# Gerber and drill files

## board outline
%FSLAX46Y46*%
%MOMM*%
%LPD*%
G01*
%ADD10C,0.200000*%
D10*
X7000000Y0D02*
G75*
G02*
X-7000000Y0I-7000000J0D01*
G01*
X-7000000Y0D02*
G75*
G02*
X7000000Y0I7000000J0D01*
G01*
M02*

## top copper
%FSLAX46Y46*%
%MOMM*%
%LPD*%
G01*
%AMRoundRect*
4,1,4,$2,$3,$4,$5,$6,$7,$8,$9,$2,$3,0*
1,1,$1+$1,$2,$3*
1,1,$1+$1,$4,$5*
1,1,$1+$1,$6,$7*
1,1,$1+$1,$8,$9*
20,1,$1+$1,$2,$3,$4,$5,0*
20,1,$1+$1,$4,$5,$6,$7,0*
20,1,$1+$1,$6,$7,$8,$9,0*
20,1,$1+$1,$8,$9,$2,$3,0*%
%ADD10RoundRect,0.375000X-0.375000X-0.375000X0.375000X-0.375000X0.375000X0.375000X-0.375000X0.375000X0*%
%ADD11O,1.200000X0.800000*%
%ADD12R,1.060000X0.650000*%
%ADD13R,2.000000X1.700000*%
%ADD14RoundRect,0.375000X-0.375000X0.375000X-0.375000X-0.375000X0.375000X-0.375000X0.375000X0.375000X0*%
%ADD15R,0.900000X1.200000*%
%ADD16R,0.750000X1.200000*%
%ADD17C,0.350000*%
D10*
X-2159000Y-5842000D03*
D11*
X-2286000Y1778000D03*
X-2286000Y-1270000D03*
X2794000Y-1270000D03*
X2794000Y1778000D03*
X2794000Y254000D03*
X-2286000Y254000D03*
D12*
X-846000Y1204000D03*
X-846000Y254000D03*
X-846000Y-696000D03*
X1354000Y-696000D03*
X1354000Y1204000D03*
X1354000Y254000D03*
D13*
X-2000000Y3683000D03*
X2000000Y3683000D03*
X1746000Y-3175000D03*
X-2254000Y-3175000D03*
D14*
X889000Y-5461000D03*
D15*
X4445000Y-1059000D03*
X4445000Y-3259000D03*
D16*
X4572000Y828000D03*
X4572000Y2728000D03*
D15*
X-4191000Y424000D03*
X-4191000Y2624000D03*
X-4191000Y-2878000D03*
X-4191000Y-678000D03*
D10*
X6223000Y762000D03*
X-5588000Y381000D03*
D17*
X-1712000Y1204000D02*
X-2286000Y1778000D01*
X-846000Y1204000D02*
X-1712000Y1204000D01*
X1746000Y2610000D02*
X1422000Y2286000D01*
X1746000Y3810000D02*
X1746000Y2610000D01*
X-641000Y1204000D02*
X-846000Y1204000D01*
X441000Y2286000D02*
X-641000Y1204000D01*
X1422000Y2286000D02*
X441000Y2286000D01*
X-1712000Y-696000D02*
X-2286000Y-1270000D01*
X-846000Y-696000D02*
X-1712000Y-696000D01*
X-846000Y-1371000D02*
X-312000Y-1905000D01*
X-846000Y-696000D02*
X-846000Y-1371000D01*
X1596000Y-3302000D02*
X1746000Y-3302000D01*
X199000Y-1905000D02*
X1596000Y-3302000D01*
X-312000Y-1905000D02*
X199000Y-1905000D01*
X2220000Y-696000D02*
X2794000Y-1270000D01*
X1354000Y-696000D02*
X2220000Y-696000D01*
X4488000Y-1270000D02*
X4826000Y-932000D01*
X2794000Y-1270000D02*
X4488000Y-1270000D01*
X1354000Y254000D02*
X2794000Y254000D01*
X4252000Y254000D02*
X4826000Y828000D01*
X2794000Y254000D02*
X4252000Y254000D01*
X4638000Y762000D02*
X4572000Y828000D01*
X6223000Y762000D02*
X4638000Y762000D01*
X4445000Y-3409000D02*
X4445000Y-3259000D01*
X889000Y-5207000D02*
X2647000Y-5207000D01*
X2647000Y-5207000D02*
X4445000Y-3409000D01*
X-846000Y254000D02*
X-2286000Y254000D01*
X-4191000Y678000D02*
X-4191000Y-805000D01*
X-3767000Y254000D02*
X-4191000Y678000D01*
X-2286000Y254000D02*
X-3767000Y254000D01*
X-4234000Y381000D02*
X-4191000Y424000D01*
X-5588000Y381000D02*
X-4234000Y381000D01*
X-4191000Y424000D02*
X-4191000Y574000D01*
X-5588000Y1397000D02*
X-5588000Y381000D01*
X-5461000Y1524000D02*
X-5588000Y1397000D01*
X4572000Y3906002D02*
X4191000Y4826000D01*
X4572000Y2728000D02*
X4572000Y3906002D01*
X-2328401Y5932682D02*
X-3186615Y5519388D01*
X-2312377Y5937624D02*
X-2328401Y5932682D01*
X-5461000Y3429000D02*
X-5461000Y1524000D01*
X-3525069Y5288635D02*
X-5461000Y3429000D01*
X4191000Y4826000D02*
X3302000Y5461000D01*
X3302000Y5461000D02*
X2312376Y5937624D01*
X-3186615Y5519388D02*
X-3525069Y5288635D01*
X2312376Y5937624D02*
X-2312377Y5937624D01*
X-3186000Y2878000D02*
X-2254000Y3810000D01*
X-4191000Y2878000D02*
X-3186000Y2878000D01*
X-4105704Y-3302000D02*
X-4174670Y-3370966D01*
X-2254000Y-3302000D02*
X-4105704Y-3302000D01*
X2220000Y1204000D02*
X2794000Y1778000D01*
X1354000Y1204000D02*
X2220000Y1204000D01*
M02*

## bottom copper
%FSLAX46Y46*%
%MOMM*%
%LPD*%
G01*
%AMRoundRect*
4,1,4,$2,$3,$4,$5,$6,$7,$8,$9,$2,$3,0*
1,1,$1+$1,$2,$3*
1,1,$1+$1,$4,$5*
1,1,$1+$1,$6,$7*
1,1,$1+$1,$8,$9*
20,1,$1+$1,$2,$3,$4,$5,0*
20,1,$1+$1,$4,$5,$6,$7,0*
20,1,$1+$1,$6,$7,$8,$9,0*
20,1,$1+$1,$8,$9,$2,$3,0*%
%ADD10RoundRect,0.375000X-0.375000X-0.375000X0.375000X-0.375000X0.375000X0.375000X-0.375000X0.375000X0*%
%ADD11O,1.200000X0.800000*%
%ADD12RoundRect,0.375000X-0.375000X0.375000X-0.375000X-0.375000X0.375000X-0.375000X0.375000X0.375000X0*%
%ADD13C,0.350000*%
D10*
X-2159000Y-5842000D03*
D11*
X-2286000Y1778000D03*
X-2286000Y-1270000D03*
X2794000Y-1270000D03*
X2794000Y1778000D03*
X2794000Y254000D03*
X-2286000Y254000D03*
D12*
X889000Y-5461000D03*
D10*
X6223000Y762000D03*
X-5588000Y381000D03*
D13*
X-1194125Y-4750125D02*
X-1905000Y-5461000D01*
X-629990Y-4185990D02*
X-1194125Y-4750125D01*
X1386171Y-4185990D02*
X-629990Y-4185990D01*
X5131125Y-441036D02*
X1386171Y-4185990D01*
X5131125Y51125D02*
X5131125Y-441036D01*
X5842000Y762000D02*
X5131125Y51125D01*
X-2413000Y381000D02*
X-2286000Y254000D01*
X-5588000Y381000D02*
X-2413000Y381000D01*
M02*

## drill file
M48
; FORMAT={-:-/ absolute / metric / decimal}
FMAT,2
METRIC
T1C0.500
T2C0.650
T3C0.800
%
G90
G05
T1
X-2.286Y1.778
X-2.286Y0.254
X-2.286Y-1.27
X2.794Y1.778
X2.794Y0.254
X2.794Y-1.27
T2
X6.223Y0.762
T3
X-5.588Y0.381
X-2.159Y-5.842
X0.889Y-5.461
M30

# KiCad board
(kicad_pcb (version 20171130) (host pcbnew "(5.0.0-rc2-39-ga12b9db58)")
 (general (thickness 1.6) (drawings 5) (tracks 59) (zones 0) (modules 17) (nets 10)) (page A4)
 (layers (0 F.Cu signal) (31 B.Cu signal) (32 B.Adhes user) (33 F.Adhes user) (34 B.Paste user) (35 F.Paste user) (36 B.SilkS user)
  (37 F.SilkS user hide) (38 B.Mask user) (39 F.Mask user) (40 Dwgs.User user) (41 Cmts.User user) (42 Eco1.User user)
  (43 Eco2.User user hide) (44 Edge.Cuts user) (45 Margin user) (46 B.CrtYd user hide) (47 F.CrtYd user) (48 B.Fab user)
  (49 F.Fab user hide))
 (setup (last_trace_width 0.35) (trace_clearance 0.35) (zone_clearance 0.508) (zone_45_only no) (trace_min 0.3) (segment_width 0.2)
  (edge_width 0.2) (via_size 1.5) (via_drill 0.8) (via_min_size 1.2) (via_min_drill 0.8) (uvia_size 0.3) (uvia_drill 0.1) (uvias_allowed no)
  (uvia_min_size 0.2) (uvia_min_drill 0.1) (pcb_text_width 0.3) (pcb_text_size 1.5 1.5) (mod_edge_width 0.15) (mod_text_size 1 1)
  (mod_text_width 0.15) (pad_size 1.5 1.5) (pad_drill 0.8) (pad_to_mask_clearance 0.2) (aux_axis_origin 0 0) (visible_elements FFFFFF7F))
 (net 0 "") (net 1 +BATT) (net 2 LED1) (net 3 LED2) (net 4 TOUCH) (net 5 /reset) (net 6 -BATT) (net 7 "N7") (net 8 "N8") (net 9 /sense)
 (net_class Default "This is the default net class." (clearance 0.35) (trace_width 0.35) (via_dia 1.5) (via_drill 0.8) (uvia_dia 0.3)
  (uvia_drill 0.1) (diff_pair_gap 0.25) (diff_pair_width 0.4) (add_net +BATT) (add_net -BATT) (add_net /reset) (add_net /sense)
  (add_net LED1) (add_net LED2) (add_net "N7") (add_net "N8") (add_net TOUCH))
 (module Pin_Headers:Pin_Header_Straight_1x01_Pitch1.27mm (layer F.Cu) (at -2.159 5.842)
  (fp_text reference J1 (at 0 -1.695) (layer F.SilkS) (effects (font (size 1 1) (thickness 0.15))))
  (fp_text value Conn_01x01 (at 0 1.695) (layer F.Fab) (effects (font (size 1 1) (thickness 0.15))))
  (pad 1 thru_hole roundrect (at 0 0) (size 1.5 1.5) (drill 0.8) (layers *.Cu *.Mask) (roundrect_rratio 0.25) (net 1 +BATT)))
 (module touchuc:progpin (layer F.Cu) (at -2.286 -1.778 90)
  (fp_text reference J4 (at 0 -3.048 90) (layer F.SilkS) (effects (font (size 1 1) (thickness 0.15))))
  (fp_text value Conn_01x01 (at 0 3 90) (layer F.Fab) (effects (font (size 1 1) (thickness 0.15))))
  (pad 1 thru_hole oval (at 0 0 90) (size 0.8 1.2) (drill 0.5) (layers *.Cu *.Mask) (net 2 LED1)))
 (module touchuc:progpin (layer F.Cu) (at -2.286 1.27 90)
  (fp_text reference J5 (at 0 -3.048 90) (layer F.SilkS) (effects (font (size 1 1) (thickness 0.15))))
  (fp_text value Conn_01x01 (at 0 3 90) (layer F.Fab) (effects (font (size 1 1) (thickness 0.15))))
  (pad 1 thru_hole oval (at 0 0 90) (size 0.8 1.2) (drill 0.5) (layers *.Cu *.Mask) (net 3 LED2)))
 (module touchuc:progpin (layer F.Cu) (at 2.794 1.27 90)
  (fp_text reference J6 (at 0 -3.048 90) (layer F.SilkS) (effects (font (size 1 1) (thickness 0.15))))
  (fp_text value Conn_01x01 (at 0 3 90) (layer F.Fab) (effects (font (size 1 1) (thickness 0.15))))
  (pad 1 thru_hole oval (at 0 0 90) (size 0.8 1.2) (drill 0.5) (layers *.Cu *.Mask) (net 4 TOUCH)))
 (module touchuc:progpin (layer F.Cu) (at 2.794 -1.778 90)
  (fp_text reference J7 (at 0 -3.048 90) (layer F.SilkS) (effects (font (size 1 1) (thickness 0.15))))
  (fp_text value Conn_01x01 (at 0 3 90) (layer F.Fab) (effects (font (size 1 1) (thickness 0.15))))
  (pad 1 thru_hole oval (at 0 0 90) (size 0.8 1.2) (drill 0.5) (layers *.Cu *.Mask) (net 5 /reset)))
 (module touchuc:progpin (layer F.Cu) (at 2.794 -0.254 90)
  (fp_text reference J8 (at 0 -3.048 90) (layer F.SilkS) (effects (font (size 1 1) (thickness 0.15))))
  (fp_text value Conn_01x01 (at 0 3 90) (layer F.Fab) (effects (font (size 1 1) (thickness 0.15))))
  (pad 1 thru_hole oval (at 0 0 90) (size 0.8 1.2) (drill 0.5) (layers *.Cu *.Mask) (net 1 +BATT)))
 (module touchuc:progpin (layer F.Cu) (at -2.286 -0.254 90)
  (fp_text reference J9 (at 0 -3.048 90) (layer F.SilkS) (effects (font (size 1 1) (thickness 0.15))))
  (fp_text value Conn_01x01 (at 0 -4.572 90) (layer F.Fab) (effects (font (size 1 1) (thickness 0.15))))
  (pad 1 thru_hole oval (at 0 0 90) (size 0.8 1.2) (drill 0.5) (layers *.Cu *.Mask) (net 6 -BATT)))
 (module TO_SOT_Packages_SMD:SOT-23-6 (layer F.Cu) (at 0.254 -0.254)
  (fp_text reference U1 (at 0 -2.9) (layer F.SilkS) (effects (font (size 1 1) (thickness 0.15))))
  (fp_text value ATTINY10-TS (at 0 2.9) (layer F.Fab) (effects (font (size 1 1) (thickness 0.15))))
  (pad 1 smd rect (at -1.1 -0.95) (size 1.06 0.65) (layers F.Cu F.Paste F.Mask) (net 2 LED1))
  (pad 2 smd rect (at -1.1 0) (size 1.06 0.65) (layers F.Cu F.Paste F.Mask) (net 6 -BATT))
  (pad 3 smd rect (at -1.1 0.95) (size 1.06 0.65) (layers F.Cu F.Paste F.Mask) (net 3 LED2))
  (pad 4 smd rect (at 1.1 0.95) (size 1.06 0.65) (layers F.Cu F.Paste F.Mask) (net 4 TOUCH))
  (pad 6 smd rect (at 1.1 -0.95) (size 1.06 0.65) (layers F.Cu F.Paste F.Mask) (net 5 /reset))
  (pad 5 smd rect (at 1.1 0) (size 1.06 0.65) (layers F.Cu F.Paste F.Mask) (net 1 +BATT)))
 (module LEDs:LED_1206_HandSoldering (layer F.Cu) (at 0 -3.683)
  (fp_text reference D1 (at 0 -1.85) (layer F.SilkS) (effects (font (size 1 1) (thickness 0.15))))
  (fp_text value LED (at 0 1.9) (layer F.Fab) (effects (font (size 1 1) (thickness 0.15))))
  (pad 1 smd rect (at -2 0) (size 2 1.7) (layers F.Cu F.Paste F.Mask) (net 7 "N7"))
  (pad 2 smd rect (at 2 0) (size 2 1.7) (layers F.Cu F.Paste F.Mask) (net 2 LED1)))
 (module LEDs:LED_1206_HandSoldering (layer F.Cu) (at -0.254 3.175)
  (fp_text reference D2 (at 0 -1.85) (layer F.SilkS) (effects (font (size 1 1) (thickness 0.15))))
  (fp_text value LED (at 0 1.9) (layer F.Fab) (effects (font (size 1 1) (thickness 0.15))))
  (pad 2 smd rect (at 2 0) (size 2 1.7) (layers F.Cu F.Paste F.Mask) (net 3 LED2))
  (pad 1 smd rect (at -2 0) (size 2 1.7) (layers F.Cu F.Paste F.Mask) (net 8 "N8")))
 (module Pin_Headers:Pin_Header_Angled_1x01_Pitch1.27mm (layer F.Cu) (at 0.889 5.461 270)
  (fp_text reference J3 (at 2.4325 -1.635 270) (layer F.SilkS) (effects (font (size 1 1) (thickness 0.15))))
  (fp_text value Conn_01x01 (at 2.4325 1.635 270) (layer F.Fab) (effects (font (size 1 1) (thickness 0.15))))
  (pad 1 thru_hole roundrect (at 0 0 270) (size 1.5 1.5) (drill 0.8) (layers *.Cu *.Mask) (roundrect_rratio 0.25) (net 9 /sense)))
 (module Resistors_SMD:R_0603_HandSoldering (layer F.Cu) (at 4.445 2.159 270)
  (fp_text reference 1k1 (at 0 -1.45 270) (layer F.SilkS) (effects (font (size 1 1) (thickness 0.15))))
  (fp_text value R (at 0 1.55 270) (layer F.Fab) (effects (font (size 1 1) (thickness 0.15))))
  (pad 1 smd rect (at -1.1 0 270) (size 1.2 0.9) (layers F.Cu F.Paste F.Mask) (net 4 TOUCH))
  (pad 2 smd rect (at 1.1 0 270) (size 1.2 0.9) (layers F.Cu F.Paste F.Mask) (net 9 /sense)))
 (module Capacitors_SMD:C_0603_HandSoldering (layer F.Cu) (at 4.572 -1.778 90)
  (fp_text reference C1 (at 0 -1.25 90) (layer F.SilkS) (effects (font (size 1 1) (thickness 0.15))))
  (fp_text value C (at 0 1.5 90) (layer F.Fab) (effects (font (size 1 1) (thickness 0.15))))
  (pad 1 smd rect (at -0.95 0 90) (size 1.2 0.75) (layers F.Cu F.Paste F.Mask) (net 1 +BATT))
  (pad 2 smd rect (at 0.95 0 90) (size 1.2 0.75) (layers F.Cu F.Paste F.Mask) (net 6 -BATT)))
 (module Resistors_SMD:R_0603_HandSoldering (layer F.Cu) (at -4.191 -1.524 270)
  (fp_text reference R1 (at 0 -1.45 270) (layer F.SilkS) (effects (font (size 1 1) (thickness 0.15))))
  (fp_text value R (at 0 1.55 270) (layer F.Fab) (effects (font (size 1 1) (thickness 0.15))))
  (pad 2 smd rect (at 1.1 0 270) (size 1.2 0.9) (layers F.Cu F.Paste F.Mask) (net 6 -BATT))
  (pad 1 smd rect (at -1.1 0 270) (size 1.2 0.9) (layers F.Cu F.Paste F.Mask) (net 7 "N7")))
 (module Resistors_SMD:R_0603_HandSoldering (layer F.Cu) (at -4.191 1.778 90)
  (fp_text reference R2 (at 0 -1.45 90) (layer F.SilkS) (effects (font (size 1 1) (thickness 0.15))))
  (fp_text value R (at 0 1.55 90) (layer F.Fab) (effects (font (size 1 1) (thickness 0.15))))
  (pad 1 smd rect (at -1.1 0 90) (size 1.2 0.9) (layers F.Cu F.Paste F.Mask) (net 8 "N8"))
  (pad 2 smd rect (at 1.1 0 90) (size 1.2 0.9) (layers F.Cu F.Paste F.Mask) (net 6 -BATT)))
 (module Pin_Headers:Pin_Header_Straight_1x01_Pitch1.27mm (layer F.Cu) (at 6.223 -0.762)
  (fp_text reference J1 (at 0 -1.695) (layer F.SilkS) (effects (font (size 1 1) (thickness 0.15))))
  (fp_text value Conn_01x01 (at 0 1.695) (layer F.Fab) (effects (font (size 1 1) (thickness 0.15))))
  (pad 1 thru_hole roundrect (at 0 0) (size 1.5 1.5) (drill 0.65) (layers *.Cu *.Mask) (roundrect_rratio 0.25) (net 1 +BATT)))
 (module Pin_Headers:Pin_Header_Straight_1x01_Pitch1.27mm (layer F.Cu) (at -5.588 -0.381)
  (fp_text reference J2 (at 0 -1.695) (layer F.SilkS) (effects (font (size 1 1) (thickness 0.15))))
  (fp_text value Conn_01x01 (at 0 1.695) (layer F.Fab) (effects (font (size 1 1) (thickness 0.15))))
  (pad 1 thru_hole roundrect (at 0 0) (size 1.5 1.5) (drill 0.8) (layers *.Cu *.Mask) (roundrect_rratio 0.25) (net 6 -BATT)))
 (gr_circle (center 0 0) (end 7 0) (layer Edge.Cuts) (width 0.2))
 (segment (start -1.712 -1.204) (end -2.286 -1.778) (width 0.35) (layer F.Cu) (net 2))
 (segment (start -0.846 -1.204) (end -1.712 -1.204) (width 0.35) (layer F.Cu) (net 2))
 (segment (start 1.746 -2.61) (end 1.422 -2.286) (width 0.35) (layer F.Cu) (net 2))
 (segment (start 1.746 -3.81) (end 1.746 -2.61) (width 0.35) (layer F.Cu) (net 2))
 (segment (start -0.641 -1.204) (end -0.846 -1.204) (width 0.35) (layer F.Cu) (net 2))
 (segment (start 0.441 -2.286) (end -0.641 -1.204) (width 0.35) (layer F.Cu) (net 2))
 (segment (start 1.422 -2.286) (end 0.441 -2.286) (width 0.35) (layer F.Cu) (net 2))
 (segment (start -1.712 0.696) (end -2.286 1.27) (width 0.35) (layer F.Cu) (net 3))
 (segment (start -0.846 0.696) (end -1.712 0.696) (width 0.35) (layer F.Cu) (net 3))
 (segment (start -0.846 1.371) (end -0.312 1.905) (width 0.35) (layer F.Cu) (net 3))
 (segment (start -0.846 0.696) (end -0.846 1.371) (width 0.35) (layer F.Cu) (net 3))
 (segment (start 1.596 3.302) (end 1.746 3.302) (width 0.35) (layer F.Cu) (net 3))
 (segment (start 0.199 1.905) (end 1.596 3.302) (width 0.35) (layer F.Cu) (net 3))
 (segment (start -0.312 1.905) (end 0.199 1.905) (width 0.35) (layer F.Cu) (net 3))
 (segment (start 2.22 0.696) (end 2.794 1.27) (width 0.35) (layer F.Cu) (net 4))
 (segment (start 1.354 0.696) (end 2.22 0.696) (width 0.35) (layer F.Cu) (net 4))
 (segment (start 4.488 1.27) (end 4.826 0.932) (width 0.35) (layer F.Cu) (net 4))
 (segment (start 2.794 1.27) (end 4.488 1.27) (width 0.35) (layer F.Cu) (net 4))
 (segment (start 1.354 -0.254) (end 2.794 -0.254) (width 0.35) (layer F.Cu) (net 1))
 (segment (start 4.252 -0.254) (end 4.826 -0.828) (width 0.35) (layer F.Cu) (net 1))
 (segment (start 2.794 -0.254) (end 4.252 -0.254) (width 0.35) (layer F.Cu) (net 1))
 (segment (start 4.638 -0.762) (end 4.572 -0.828) (width 0.35) (layer F.Cu) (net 1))
 (segment (start 6.223 -0.762) (end 4.638 -0.762) (width 0.35) (layer F.Cu) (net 1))
 (segment (start -1.194125 4.750125) (end -1.905 5.461) (width 0.35) (layer B.Cu) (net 1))
 (segment (start -0.62999 4.18599) (end -1.194125 4.750125) (width 0.35) (layer B.Cu) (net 1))
 (segment (start 1.386171 4.18599) (end -0.62999 4.18599) (width 0.35) (layer B.Cu) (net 1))
 (segment (start 5.131125 0.441036) (end 1.386171 4.18599) (width 0.35) (layer B.Cu) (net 1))
 (segment (start 5.131125 -0.051125) (end 5.131125 0.441036) (width 0.35) (layer B.Cu) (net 1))
 (segment (start 5.842 -0.762) (end 5.131125 -0.051125) (width 0.35) (layer B.Cu) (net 1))
 (segment (start 4.445 3.409) (end 4.445 3.259) (width 0.35) (layer F.Cu) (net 9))
 (segment (start 0.889 5.207) (end 2.647 5.207) (width 0.35) (layer F.Cu) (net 9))
 (segment (start 2.647 5.207) (end 4.445 3.409) (width 0.35) (layer F.Cu) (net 9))
 (segment (start -0.846 -0.254) (end -2.286 -0.254) (width 0.35) (layer F.Cu) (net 6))
 (segment (start -4.191 -0.678) (end -4.191 0.805) (width 0.35) (layer F.Cu) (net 6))
 (segment (start -3.767 -0.254) (end -4.191 -0.678) (width 0.35) (layer F.Cu) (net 6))
 (segment (start -2.286 -0.254) (end -3.767 -0.254) (width 0.35) (layer F.Cu) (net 6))
 (segment (start -4.234 -0.381) (end -4.191 -0.424) (width 0.35) (layer F.Cu) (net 6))
 (segment (start -5.588 -0.381) (end -4.234 -0.381) (width 0.35) (layer F.Cu) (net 6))
 (segment (start -4.191 -0.424) (end -4.191 -0.574) (width 0.35) (layer F.Cu) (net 6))
 (segment (start -5.588 -1.397) (end -5.588 -0.381) (width 0.35) (layer F.Cu) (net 6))
 (segment (start -5.461 -1.524) (end -5.588 -1.397) (width 0.35) (layer F.Cu) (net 6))
 (segment (start 4.572 -3.906002) (end 4.191 -4.826) (width 0.35) (layer F.Cu) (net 6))
 (segment (start 4.572 -2.728) (end 4.572 -3.906002) (width 0.35) (layer F.Cu) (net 6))
 (segment (start -2.328401 -5.932682) (end -3.186615 -5.519388) (width 0.35) (layer F.Cu) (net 6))
 (segment (start -2.312377 -5.937624) (end -2.328401 -5.932682) (width 0.35) (layer F.Cu) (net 6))
 (segment (start -5.461 -3.429) (end -5.461 -1.524) (width 0.35) (layer F.Cu) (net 6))
 (segment (start -3.525069 -5.288635) (end -5.461 -3.429) (width 0.35) (layer F.Cu) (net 6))
 (segment (start 4.191 -4.826) (end 3.302 -5.461) (width 0.35) (layer F.Cu) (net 6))
 (segment (start 3.302 -5.461) (end 2.312376 -5.937624) (width 0.35) (layer F.Cu) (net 6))
 (segment (start -3.186615 -5.519388) (end -3.525069 -5.288635) (width 0.35) (layer F.Cu) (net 6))
 (segment (start 2.312376 -5.937624) (end -2.312377 -5.937624) (width 0.35) (layer F.Cu) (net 6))
 (segment (start -2.413 -0.381) (end -2.286 -0.254) (width 0.35) (layer B.Cu) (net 6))
 (segment (start -5.588 -0.381) (end -2.413 -0.381) (width 0.35) (layer B.Cu) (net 6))
 (segment (start -3.186 -2.878) (end -2.254 -3.81) (width 0.35) (layer F.Cu) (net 7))
 (segment (start -4.191 -2.878) (end -3.186 -2.878) (width 0.35) (layer F.Cu) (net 7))
 (segment (start -4.105704 3.302) (end -4.17467 3.370966) (width 0.35) (layer F.Cu) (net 8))
 (segment (start -2.254 3.302) (end -4.105704 3.302) (width 0.35) (layer F.Cu) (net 8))
 (segment (start 2.22 -1.204) (end 2.794 -1.778) (width 0.35) (layer F.Cu) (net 5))
 (segment (start 1.354 -1.204) (end 2.22 -1.204) (width 0.35) (layer F.Cu) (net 5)))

